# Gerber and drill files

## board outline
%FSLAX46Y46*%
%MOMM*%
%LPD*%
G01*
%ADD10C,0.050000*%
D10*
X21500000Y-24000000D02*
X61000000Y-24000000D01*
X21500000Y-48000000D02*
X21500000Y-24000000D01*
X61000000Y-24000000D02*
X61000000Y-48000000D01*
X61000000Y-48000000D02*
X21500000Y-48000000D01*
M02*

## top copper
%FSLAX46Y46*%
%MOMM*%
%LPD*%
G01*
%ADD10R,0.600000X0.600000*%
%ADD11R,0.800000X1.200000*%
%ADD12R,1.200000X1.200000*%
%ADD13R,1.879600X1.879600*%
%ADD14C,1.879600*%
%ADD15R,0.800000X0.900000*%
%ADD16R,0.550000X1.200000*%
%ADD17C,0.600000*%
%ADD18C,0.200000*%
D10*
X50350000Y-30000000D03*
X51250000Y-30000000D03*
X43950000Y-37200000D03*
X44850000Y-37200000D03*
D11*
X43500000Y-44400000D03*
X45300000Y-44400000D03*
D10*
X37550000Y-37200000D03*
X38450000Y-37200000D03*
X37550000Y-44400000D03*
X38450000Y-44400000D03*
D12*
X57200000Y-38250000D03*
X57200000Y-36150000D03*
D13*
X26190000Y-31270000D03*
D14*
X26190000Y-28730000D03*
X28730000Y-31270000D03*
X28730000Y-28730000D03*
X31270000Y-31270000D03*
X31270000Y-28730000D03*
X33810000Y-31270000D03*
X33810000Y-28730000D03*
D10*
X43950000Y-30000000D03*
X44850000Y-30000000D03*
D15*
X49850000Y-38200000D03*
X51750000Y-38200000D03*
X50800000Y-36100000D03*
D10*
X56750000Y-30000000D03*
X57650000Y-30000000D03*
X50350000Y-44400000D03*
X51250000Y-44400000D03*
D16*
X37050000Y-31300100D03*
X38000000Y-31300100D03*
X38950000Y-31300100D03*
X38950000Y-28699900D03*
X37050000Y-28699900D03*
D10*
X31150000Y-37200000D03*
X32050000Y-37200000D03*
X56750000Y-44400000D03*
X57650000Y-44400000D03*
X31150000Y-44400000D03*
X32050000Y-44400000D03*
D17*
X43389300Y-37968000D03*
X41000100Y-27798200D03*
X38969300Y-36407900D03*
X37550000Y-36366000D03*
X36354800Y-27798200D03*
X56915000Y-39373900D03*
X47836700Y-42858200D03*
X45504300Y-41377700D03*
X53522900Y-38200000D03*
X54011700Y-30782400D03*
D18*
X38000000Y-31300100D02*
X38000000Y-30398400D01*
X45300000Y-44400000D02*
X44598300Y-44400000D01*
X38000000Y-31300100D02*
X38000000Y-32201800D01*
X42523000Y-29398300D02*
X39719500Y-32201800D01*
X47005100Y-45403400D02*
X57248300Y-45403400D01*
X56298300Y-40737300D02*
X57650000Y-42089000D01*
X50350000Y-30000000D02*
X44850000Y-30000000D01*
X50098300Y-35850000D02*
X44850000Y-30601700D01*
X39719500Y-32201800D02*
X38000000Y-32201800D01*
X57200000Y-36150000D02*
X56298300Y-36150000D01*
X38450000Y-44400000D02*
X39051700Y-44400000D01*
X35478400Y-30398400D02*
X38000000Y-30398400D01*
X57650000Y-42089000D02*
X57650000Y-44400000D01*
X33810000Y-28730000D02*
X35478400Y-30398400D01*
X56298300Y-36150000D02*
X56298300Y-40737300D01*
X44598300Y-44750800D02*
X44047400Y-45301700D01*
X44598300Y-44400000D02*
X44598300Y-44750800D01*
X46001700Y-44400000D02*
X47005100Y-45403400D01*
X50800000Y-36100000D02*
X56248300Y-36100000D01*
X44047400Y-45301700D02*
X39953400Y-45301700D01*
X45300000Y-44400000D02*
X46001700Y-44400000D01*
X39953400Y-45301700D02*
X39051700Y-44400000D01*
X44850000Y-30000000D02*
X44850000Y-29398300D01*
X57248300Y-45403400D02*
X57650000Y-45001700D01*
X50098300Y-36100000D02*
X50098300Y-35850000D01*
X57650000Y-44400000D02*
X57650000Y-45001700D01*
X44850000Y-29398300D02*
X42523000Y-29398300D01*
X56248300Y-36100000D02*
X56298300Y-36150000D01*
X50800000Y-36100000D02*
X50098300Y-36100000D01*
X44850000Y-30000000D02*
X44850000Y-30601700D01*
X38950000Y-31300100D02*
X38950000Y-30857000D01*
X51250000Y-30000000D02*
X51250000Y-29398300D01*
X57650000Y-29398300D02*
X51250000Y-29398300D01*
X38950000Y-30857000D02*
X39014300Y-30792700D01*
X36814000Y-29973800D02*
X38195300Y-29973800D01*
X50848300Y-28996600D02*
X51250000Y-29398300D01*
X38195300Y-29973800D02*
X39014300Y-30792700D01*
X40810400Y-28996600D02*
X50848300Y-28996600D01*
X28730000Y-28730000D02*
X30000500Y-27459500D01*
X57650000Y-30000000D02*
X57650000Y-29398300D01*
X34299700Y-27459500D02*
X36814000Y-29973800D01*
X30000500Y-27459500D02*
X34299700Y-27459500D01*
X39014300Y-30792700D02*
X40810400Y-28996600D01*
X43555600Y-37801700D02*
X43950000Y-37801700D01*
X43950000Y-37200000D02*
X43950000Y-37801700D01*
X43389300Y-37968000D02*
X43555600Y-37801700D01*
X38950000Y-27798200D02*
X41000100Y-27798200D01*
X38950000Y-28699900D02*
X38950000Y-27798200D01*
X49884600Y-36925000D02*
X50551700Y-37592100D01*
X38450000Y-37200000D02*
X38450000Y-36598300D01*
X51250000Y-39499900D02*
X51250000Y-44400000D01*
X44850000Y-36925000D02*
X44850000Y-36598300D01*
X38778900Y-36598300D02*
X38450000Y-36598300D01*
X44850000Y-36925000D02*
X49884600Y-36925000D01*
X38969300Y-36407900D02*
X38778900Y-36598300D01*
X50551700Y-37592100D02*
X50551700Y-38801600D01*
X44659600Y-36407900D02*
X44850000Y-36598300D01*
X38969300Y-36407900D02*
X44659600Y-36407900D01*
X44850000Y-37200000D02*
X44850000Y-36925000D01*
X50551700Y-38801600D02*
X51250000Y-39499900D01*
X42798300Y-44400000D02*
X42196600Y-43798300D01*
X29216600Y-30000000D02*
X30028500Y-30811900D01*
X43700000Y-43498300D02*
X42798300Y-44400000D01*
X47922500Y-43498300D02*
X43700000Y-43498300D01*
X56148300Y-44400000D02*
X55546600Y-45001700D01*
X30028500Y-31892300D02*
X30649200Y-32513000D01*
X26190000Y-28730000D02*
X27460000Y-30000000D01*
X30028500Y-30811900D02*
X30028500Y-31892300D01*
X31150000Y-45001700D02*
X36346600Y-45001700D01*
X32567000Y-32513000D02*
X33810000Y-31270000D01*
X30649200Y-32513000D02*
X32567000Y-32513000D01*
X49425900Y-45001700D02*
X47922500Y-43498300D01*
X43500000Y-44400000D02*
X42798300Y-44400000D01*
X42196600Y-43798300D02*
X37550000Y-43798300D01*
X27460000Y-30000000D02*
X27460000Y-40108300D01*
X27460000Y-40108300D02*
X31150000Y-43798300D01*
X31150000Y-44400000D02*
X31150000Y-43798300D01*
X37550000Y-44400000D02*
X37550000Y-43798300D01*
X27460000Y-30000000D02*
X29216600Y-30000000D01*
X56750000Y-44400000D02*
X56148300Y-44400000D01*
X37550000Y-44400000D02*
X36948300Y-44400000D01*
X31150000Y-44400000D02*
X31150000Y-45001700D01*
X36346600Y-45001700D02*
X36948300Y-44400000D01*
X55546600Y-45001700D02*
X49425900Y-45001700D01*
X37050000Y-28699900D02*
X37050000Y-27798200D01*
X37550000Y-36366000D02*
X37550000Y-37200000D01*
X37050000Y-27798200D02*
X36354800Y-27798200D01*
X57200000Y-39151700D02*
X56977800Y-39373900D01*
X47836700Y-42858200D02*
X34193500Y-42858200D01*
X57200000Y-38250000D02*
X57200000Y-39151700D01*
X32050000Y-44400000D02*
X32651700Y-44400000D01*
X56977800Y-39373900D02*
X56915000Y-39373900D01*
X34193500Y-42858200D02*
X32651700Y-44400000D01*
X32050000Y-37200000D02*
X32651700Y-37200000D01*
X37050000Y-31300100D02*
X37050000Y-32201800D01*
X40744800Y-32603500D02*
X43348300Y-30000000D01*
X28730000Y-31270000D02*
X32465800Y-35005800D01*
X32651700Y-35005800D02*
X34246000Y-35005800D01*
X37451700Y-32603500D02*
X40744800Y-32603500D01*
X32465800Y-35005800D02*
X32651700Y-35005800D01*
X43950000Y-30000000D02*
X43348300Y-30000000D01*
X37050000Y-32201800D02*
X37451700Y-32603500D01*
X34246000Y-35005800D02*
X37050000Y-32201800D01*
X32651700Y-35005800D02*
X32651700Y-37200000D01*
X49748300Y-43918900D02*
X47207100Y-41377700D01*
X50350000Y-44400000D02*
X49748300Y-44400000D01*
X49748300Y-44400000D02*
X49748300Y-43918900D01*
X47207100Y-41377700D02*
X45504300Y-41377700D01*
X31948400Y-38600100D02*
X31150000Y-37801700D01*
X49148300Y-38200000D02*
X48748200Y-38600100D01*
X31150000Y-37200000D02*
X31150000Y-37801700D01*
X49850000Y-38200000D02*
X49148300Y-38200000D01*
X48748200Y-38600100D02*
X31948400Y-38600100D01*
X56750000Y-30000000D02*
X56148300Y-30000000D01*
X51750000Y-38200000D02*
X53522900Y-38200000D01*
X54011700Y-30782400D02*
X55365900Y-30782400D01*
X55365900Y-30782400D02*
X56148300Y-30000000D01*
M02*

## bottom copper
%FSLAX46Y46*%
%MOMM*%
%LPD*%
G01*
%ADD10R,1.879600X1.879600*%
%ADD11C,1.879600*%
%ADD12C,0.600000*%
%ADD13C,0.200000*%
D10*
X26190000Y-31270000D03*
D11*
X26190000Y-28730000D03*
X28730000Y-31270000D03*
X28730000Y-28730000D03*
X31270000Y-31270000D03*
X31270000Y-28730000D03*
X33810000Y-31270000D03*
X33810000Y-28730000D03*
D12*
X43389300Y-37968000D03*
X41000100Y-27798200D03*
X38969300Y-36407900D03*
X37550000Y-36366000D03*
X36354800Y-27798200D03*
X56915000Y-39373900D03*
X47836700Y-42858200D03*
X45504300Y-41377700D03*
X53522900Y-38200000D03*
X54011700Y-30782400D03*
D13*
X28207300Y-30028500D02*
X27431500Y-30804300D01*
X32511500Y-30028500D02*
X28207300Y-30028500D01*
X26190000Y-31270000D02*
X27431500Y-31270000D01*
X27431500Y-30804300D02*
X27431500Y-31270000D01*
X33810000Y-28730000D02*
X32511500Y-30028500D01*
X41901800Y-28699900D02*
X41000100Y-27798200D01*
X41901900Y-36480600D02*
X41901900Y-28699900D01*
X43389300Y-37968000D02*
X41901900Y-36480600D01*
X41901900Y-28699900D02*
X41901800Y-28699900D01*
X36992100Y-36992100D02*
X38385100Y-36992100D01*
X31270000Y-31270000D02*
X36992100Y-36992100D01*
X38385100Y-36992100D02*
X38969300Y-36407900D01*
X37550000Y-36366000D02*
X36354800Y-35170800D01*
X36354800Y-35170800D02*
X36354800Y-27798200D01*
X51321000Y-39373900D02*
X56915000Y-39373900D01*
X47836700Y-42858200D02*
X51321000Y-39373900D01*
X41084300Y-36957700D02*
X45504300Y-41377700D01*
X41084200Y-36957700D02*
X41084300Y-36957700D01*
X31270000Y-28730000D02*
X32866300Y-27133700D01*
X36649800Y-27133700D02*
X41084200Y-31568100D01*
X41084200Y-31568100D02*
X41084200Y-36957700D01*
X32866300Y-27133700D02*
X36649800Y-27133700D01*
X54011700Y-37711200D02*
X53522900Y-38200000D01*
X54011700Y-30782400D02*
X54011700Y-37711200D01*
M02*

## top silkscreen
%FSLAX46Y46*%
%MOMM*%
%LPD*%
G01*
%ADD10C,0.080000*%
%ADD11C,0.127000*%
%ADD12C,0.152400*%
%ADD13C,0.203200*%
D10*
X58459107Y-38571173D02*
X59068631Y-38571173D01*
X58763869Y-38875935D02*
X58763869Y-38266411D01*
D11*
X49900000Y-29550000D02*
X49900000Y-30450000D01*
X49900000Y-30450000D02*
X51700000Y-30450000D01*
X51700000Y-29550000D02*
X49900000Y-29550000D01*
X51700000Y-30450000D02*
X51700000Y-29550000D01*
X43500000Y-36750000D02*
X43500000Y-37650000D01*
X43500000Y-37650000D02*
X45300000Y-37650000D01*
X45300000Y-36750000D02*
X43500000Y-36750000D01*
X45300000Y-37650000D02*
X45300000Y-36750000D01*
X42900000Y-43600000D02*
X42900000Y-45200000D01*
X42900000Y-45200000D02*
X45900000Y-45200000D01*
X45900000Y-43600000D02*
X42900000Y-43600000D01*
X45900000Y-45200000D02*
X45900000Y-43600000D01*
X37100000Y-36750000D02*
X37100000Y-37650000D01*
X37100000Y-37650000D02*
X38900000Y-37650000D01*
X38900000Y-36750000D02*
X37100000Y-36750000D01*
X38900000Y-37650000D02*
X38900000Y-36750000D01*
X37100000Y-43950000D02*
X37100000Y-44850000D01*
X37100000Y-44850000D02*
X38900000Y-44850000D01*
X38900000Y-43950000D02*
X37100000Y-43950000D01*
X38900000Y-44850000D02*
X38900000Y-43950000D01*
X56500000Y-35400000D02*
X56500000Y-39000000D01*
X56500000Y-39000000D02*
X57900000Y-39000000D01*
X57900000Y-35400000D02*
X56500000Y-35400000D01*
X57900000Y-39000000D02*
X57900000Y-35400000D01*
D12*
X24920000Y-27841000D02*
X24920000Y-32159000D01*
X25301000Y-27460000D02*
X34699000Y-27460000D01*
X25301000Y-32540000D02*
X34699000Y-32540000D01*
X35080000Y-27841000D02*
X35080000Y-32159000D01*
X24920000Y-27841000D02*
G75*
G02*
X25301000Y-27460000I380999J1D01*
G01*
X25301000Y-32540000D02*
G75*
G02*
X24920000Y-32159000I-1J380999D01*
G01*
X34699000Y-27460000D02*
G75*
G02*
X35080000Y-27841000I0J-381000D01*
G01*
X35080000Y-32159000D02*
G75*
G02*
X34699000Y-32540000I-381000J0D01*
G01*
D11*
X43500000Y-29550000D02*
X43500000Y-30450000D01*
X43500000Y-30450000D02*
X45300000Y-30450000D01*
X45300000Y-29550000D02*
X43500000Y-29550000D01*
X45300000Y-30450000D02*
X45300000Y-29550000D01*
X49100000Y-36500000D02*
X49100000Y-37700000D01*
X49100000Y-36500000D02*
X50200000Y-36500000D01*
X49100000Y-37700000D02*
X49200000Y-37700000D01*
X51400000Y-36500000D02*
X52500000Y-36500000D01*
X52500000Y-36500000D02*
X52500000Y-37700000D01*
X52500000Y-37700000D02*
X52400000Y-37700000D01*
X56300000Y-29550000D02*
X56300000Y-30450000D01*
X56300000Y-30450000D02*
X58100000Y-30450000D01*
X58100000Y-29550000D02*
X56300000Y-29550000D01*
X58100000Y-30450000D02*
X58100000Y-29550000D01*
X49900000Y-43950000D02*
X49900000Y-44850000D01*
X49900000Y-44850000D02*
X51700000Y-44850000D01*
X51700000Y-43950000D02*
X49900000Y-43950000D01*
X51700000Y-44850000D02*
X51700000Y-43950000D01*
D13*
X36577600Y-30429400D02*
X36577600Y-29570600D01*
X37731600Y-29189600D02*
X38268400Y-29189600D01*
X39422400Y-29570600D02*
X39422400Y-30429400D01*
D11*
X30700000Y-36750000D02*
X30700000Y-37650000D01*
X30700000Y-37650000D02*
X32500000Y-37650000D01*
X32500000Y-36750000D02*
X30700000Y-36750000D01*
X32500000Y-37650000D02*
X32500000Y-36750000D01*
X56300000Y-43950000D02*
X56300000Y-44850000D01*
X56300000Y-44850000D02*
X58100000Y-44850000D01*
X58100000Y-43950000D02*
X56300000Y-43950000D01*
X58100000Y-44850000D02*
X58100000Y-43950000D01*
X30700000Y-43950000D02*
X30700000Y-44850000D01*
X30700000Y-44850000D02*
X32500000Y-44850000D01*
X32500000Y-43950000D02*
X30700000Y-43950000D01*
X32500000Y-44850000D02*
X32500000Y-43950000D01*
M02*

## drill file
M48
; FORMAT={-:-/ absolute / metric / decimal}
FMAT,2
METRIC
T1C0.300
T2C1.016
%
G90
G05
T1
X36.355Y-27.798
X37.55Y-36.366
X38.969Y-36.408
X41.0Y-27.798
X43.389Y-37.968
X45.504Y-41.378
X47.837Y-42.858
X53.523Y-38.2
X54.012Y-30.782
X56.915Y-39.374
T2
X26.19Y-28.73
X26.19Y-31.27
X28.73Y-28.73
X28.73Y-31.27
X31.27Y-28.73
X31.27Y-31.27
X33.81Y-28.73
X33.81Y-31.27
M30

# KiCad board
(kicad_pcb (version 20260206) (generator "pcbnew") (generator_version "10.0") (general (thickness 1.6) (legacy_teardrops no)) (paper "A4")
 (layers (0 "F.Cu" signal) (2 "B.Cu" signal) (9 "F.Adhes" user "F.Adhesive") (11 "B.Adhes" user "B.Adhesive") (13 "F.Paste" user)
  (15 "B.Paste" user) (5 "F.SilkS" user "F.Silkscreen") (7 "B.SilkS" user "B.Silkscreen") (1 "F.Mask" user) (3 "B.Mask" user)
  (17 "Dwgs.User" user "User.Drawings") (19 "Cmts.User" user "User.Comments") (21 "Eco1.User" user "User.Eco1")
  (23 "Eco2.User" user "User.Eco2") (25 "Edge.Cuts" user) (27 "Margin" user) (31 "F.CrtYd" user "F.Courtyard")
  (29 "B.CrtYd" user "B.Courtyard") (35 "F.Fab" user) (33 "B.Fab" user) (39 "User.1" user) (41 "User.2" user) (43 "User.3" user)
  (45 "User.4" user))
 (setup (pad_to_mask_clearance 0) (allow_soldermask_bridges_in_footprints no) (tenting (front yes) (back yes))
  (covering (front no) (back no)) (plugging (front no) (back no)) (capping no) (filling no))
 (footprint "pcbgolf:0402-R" (layer "F.Cu") (at 50.8 30)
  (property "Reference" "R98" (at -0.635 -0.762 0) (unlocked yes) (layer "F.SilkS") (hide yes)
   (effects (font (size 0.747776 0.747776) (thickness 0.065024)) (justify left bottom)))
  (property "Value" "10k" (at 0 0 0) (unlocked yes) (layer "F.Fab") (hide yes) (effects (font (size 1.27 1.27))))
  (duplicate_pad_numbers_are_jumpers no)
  (fp_line (start -0.9 -0.45) (end -0.9 0.45) (stroke (width 0.127) (type solid)) (layer "F.SilkS"))
  (fp_line (start -0.9 0.45) (end 0.9 0.45) (stroke (width 0.127) (type solid)) (layer "F.SilkS"))
  (fp_line (start 0.9 -0.45) (end -0.9 -0.45) (stroke (width 0.127) (type solid)) (layer "F.SilkS"))
  (fp_line (start 0.9 0.45) (end 0.9 -0.45) (stroke (width 0.127) (type solid)) (layer "F.SilkS"))
  (pad "1" smd rect (at -0.45 0) (size 0.6 0.6) (layers "F.Cu" "F.Mask" "F.Paste") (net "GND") (solder_mask_margin 0.0508)
   (solder_paste_margin 0) (thermal_bridge_angle 0))
  (pad "2" smd rect (at 0.45 0) (size 0.6 0.6) (layers "F.Cu" "F.Mask" "F.Paste") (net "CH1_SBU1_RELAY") (solder_mask_margin 0.0508)
   (solder_paste_margin 0) (thermal_bridge_angle 0)))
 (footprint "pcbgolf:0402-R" (layer "F.Cu") (at 44.4 37.2)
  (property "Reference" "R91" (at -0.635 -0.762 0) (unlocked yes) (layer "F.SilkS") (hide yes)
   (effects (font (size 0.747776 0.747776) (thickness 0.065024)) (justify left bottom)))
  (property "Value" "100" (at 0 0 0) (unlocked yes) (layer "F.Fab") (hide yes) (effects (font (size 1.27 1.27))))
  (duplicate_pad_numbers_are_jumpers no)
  (fp_line (start -0.9 -0.45) (end -0.9 0.45) (stroke (width 0.127) (type solid)) (layer "F.SilkS"))
  (fp_line (start -0.9 0.45) (end 0.9 0.45) (stroke (width 0.127) (type solid)) (layer "F.SilkS"))
  (fp_line (start 0.9 -0.45) (end -0.9 -0.45) (stroke (width 0.127) (type solid)) (layer "F.SilkS"))
  (fp_line (start 0.9 0.45) (end 0.9 -0.45) (stroke (width 0.127) (type solid)) (layer "F.SilkS"))
  (pad "1" smd rect (at -0.45 0) (size 0.6 0.6) (layers "F.Cu" "F.Mask" "F.Paste") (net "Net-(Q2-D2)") (solder_mask_margin 0.0508)
   (solder_paste_margin 0) (thermal_bridge_angle 0))
  (pad "2" smd rect (at 0.45 0) (size 0.6 0.6) (layers "F.Cu" "F.Mask" "F.Paste") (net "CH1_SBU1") (solder_mask_margin 0.0508)
   (solder_paste_margin 0) (thermal_bridge_angle 0)))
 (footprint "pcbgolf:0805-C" (layer "F.Cu") (at 44.4 44.4)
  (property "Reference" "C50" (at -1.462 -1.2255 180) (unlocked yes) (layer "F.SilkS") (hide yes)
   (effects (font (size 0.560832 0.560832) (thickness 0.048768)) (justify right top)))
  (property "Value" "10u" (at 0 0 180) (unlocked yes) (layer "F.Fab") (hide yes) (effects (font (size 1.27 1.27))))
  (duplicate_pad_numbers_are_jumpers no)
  (fp_line (start -1.5 -0.8) (end -1.5 0.8) (stroke (width 0.127) (type solid)) (layer "F.SilkS"))
  (fp_line (start -1.5 0.8) (end 1.5 0.8) (stroke (width 0.127) (type solid)) (layer "F.SilkS"))
  (fp_line (start 1.5 -0.8) (end -1.5 -0.8) (stroke (width 0.127) (type solid)) (layer "F.SilkS"))
  (fp_line (start 1.5 0.8) (end 1.5 -0.8) (stroke (width 0.127) (type solid)) (layer "F.SilkS"))
  (pad "1" smd rect (at -0.9 0) (size 0.8 1.2) (layers "F.Cu" "F.Mask" "F.Paste") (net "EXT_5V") (solder_mask_margin 0.0508)
   (solder_paste_margin 0) (thermal_bridge_angle 0))
  (pad "2" smd rect (at 0.9 0) (size 0.8 1.2) (layers "F.Cu" "F.Mask" "F.Paste") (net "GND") (solder_mask_margin 0.0508)
   (solder_paste_margin 0) (thermal_bridge_angle 0)))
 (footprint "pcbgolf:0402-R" (layer "F.Cu") (at 38 37.2)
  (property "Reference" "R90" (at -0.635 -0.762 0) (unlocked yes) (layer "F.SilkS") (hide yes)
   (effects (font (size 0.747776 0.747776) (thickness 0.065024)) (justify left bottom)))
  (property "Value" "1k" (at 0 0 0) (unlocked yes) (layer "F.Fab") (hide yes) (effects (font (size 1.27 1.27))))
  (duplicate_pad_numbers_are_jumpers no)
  (fp_line (start -0.9 -0.45) (end -0.9 0.45) (stroke (width 0.127) (type solid)) (layer "F.SilkS"))
  (fp_line (start -0.9 0.45) (end 0.9 0.45) (stroke (width 0.127) (type solid)) (layer "F.SilkS"))
  (fp_line (start 0.9 -0.45) (end -0.9 -0.45) (stroke (width 0.127) (type solid)) (layer "F.SilkS"))
  (fp_line (start 0.9 0.45) (end 0.9 -0.45) (stroke (width 0.127) (type solid)) (layer "F.SilkS"))
  (pad "1" smd rect (at -0.45 0) (size 0.6 0.6) (layers "F.Cu" "F.Mask" "F.Paste") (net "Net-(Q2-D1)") (solder_mask_margin 0.0508)
   (solder_paste_margin 0) (thermal_bridge_angle 0))
  (pad "2" smd rect (at 0.45 0) (size 0.6 0.6) (layers "F.Cu" "F.Mask" "F.Paste") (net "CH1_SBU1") (solder_mask_margin 0.0508)
   (solder_paste_margin 0) (thermal_bridge_angle 0)))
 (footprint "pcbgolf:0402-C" (layer "F.Cu") (at 38 44.4)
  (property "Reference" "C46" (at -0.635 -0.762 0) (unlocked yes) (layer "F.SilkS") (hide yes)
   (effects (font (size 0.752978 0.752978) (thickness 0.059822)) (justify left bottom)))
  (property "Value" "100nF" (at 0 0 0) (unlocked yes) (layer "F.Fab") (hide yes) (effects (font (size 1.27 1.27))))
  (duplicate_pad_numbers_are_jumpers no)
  (fp_line (start -0.9 -0.45) (end -0.9 0.45) (stroke (width 0.127) (type solid)) (layer "F.SilkS"))
  (fp_line (start -0.9 0.45) (end 0.9 0.45) (stroke (width 0.127) (type solid)) (layer "F.SilkS"))
  (fp_line (start 0.9 -0.45) (end -0.9 -0.45) (stroke (width 0.127) (type solid)) (layer "F.SilkS"))
  (fp_line (start 0.9 0.45) (end 0.9 -0.45) (stroke (width 0.127) (type solid)) (layer "F.SilkS"))
  (pad "1" smd rect (at -0.45 0) (size 0.6 0.6) (layers "F.Cu" "F.Mask" "F.Paste") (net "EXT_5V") (solder_mask_margin 0.0508)
   (solder_paste_margin 0) (thermal_bridge_angle 0))
  (pad "2" smd rect (at 0.45 0) (size 0.6 0.6) (layers "F.Cu" "F.Mask" "F.Paste") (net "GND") (solder_mask_margin 0.0508)
   (solder_paste_margin 0) (thermal_bridge_angle 0)))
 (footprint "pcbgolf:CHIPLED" (layer "F.Cu") (at 57.2 37.2)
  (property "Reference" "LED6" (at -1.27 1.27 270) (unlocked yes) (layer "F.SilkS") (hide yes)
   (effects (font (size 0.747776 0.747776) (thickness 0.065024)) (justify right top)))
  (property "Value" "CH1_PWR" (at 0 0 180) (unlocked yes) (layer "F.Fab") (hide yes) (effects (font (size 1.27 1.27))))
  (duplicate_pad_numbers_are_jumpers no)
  (fp_line (start -0.7 -1.8) (end -0.7 1.8) (stroke (width 0.127) (type solid)) (layer "F.SilkS"))
  (fp_line (start -0.7 1.8) (end 0.7 1.8) (stroke (width 0.127) (type solid)) (layer "F.SilkS"))
  (fp_line (start 0.7 -1.8) (end -0.7 -1.8) (stroke (width 0.127) (type solid)) (layer "F.SilkS"))
  (fp_line (start 0.7 1.8) (end 0.7 -1.8) (stroke (width 0.127) (type solid)) (layer "F.SilkS"))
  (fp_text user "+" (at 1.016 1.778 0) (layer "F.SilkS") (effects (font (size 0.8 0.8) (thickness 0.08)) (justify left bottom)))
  (pad "A" smd rect (at 0 1.05) (size 1.2 1.2) (layers "F.Cu" "F.Mask" "F.Paste") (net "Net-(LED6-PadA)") (solder_mask_margin 0.0508)
   (solder_paste_margin 0) (thermal_bridge_angle 0))
  (pad "C" smd rect (at 0 -1.05) (size 1.2 1.2) (layers "F.Cu" "F.Mask" "F.Paste") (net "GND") (solder_mask_margin 0.0508)
   (solder_paste_margin 0) (thermal_bridge_angle 0)))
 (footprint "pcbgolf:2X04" (layer "F.Cu") (at 30 30)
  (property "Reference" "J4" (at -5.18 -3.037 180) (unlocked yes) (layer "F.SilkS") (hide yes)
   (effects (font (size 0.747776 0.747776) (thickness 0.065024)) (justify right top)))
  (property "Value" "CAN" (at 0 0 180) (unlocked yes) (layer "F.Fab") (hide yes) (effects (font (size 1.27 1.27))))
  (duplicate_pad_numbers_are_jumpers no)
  (fp_line (start -5.08 -2.159) (end -5.08 2.159) (stroke (width 0.1524) (type solid)) (layer "F.SilkS"))
  (fp_line (start -4.699 -2.54) (end 4.699 -2.54) (stroke (width 0.1524) (type solid)) (layer "F.SilkS"))
  (fp_line (start -4.699 2.54) (end 4.699 2.54) (stroke (width 0.1524) (type solid)) (layer "F.SilkS"))
  (fp_line (start 5.08 -2.159) (end 5.08 2.159) (stroke (width 0.1524) (type solid)) (layer "F.SilkS"))
  (fp_arc (start -5.08 -2.159) (mid -4.968408 -2.428408) (end -4.699 -2.54) (stroke (width 0.1524) (type solid)) (layer "F.SilkS"))
  (fp_arc (start -4.699 2.54) (mid -4.968408 2.428408) (end -5.08 2.159) (stroke (width 0.1524) (type solid)) (layer "F.SilkS"))
  (fp_arc (start 4.699 -2.54) (mid 4.968408 -2.428408) (end 5.08 -2.159) (stroke (width 0.1524) (type solid)) (layer "F.SilkS"))
  (fp_arc (start 5.08 2.159) (mid 4.968408 2.428408) (end 4.699 2.54) (stroke (width 0.1524) (type solid)) (layer "F.SilkS"))
  (pad "1" thru_hole rect (at -3.81 1.27 90) (size 1.8796 1.8796) (drill 1.016) (layers "*.Cu" "*.Mask") (remove_unused_layers no)
   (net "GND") (solder_mask_margin 0.0508) (thermal_bridge_angle 0))
  (pad "2" thru_hole circle (at -3.81 -1.27 90) (size 1.8796 1.8796) (drill 1.016) (layers "*.Cu" "*.Mask") (remove_unused_layers no)
   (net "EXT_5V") (solder_mask_margin 0.0508) (thermal_bridge_angle 0))
  (pad "3" thru_hole circle (at -1.27 1.27 90) (size 1.8796 1.8796) (drill 1.016) (layers "*.Cu" "*.Mask") (remove_unused_layers no)
   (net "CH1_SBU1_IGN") (solder_mask_margin 0.0508) (thermal_bridge_angle 0))
  (pad "4" thru_hole circle (at -1.27 -1.27 90) (size 1.8796 1.8796) (drill 1.016) (layers "*.Cu" "*.Mask") (remove_unused_layers no)
   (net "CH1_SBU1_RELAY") (solder_mask_margin 0.0508) (thermal_bridge_angle 0))
  (pad "5" thru_hole circle (at 1.27 1.27 90) (size 1.8796 1.8796) (drill 1.016) (layers "*.Cu" "*.Mask") (remove_unused_layers no)
   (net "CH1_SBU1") (solder_mask_margin 0.0508) (thermal_bridge_angle 0))
  (pad "6" thru_hole circle (at 1.27 -1.27 90) (size 1.8796 1.8796) (drill 1.016) (layers "*.Cu" "*.Mask") (remove_unused_layers no)
   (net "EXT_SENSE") (solder_mask_margin 0.0508) (thermal_bridge_angle 0))
  (pad "7" thru_hole circle (at 3.81 1.27 90) (size 1.8796 1.8796) (drill 1.016) (layers "*.Cu" "*.Mask") (remove_unused_layers no)
   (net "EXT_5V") (solder_mask_margin 0.0508) (thermal_bridge_angle 0))
  (pad "8" thru_hole circle (at 3.81 -1.27 90) (size 1.8796 1.8796) (drill 1.016) (layers "*.Cu" "*.Mask") (remove_unused_layers no)
   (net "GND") (solder_mask_margin 0.0508) (thermal_bridge_angle 0)))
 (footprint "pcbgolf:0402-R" (layer "F.Cu") (at 44.4 30)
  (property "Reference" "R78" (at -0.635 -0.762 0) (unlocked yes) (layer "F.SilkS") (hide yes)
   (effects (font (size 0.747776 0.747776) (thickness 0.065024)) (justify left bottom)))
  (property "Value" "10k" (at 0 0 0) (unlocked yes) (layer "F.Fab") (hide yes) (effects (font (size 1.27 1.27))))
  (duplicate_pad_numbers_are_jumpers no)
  (fp_line (start -0.9 -0.45) (end -0.9 0.45) (stroke (width 0.127) (type solid)) (layer "F.SilkS"))
  (fp_line (start -0.9 0.45) (end 0.9 0.45) (stroke (width 0.127) (type solid)) (layer "F.SilkS"))
  (fp_line (start 0.9 -0.45) (end -0.9 -0.45) (stroke (width 0.127) (type solid)) (layer "F.SilkS"))
  (fp_line (start 0.9 0.45) (end 0.9 -0.45) (stroke (width 0.127) (type solid)) (layer "F.SilkS"))
  (pad "1" smd rect (at -0.45 0) (size 0.6 0.6) (layers "F.Cu" "F.Mask" "F.Paste") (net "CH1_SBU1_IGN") (solder_mask_margin 0.0508)
   (solder_paste_margin 0) (thermal_bridge_angle 0))
  (pad "2" smd rect (at 0.45 0) (size 0.6 0.6) (layers "F.Cu" "F.Mask" "F.Paste") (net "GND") (solder_mask_margin 0.0508)
   (solder_paste_margin 0) (thermal_bridge_angle 0)))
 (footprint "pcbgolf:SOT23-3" (layer "F.Cu") (at 50.8 37.2)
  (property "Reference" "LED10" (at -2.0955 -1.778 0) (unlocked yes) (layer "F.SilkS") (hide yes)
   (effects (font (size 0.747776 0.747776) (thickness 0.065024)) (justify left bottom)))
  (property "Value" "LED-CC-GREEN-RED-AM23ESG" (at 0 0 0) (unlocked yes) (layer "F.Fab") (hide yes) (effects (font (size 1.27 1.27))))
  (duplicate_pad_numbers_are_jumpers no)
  (fp_line (start -1.7 -0.7) (end -1.7 0.5) (stroke (width 0.127) (type solid)) (layer "F.SilkS"))
  (fp_line (start -1.7 -0.7) (end -0.6 -0.7) (stroke (width 0.127) (type solid)) (layer "F.SilkS"))
  (fp_line (start -1.7 0.5) (end -1.6 0.5) (stroke (width 0.127) (type solid)) (layer "F.SilkS"))
  (fp_line (start 0.6 -0.7) (end 1.7 -0.7) (stroke (width 0.127) (type solid)) (layer "F.SilkS"))
  (fp_line (start 1.7 -0.7) (end 1.7 0.5) (stroke (width 0.127) (type solid)) (layer "F.SilkS"))
  (fp_line (start 1.7 0.5) (end 1.6 0.5) (stroke (width 0.127) (type solid)) (layer "F.SilkS"))
  (pad "1" smd rect (at -0.95 1) (size 0.8 0.9) (layers "F.Cu" "F.Mask" "F.Paste") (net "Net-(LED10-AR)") (solder_mask_margin 0.0508)
   (solder_paste_margin 0) (thermal_bridge_angle 0))
  (pad "2" smd rect (at 0.95 1) (size 0.8 0.9) (layers "F.Cu" "F.Mask" "F.Paste") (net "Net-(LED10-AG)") (solder_mask_margin 0.0508)
   (solder_paste_margin 0) (thermal_bridge_angle 0))
  (pad "3" smd rect (at 0 -1.1) (size 0.8 0.9) (layers "F.Cu" "F.Mask" "F.Paste") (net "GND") (solder_mask_margin 0.0508)
   (solder_paste_margin 0) (thermal_bridge_angle 0)))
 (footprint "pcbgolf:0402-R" (layer "F.Cu") (at 57.2 30)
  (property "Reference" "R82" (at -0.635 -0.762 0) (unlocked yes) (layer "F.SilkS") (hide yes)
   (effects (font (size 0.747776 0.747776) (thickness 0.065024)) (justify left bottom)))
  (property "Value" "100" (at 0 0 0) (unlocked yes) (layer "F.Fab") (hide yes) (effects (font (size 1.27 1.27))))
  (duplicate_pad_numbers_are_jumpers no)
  (fp_line (start -0.9 -0.45) (end -0.9 0.45) (stroke (width 0.127) (type solid)) (layer "F.SilkS"))
  (fp_line (start -0.9 0.45) (end 0.9 0.45) (stroke (width 0.127) (type solid)) (layer "F.SilkS"))
  (fp_line (start 0.9 -0.45) (end -0.9 -0.45) (stroke (width 0.127) (type solid)) (layer "F.SilkS"))
  (fp_line (start 0.9 0.45) (end 0.9 -0.45) (stroke (width 0.127) (type solid)) (layer "F.SilkS"))
  (pad "1" smd rect (at -0.45 0) (size 0.6 0.6) (layers "F.Cu" "F.Mask" "F.Paste") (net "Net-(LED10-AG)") (solder_mask_margin 0.0508)
   (solder_paste_margin 0) (thermal_bridge_angle 0))
  (pad "2" smd rect (at 0.45 0) (size 0.6 0.6) (layers "F.Cu" "F.Mask" "F.Paste") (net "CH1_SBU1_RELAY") (solder_mask_margin 0.0508)
   (solder_paste_margin 0) (thermal_bridge_angle 0)))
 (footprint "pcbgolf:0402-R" (layer "F.Cu") (at 50.8 44.4)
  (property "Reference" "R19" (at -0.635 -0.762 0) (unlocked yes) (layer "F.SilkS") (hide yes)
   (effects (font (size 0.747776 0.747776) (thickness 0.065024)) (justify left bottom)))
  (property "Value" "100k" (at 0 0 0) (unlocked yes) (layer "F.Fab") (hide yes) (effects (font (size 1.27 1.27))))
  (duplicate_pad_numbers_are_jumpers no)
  (fp_line (start -0.9 -0.45) (end -0.9 0.45) (stroke (width 0.127) (type solid)) (layer "F.SilkS"))
  (fp_line (start -0.9 0.45) (end 0.9 0.45) (stroke (width 0.127) (type solid)) (layer "F.SilkS"))
  (fp_line (start 0.9 -0.45) (end -0.9 -0.45) (stroke (width 0.127) (type solid)) (layer "F.SilkS"))
  (fp_line (start 0.9 0.45) (end 0.9 -0.45) (stroke (width 0.127) (type solid)) (layer "F.SilkS"))
  (pad "1" smd rect (at -0.45 0) (size 0.6 0.6) (layers "F.Cu" "F.Mask" "F.Paste") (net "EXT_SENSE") (solder_mask_margin 0.0508)
   (solder_paste_margin 0) (thermal_bridge_angle 0))
  (pad "2" smd rect (at 0.45 0) (size 0.6 0.6) (layers "F.Cu" "F.Mask" "F.Paste") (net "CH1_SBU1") (solder_mask_margin 0.0508)
   (solder_paste_margin 0) (thermal_bridge_angle 0)))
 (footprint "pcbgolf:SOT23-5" (layer "F.Cu") (at 38 30)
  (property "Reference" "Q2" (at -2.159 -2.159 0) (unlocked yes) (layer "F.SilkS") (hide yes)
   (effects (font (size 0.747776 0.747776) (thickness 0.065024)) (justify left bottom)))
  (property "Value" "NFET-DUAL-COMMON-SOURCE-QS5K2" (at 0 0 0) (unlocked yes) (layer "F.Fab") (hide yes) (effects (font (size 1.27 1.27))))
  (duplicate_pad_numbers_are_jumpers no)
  (fp_line (start -1.4224 0.4294) (end -1.4224 -0.4294) (stroke (width 0.2032) (type solid)) (layer "F.SilkS"))
  (fp_line (start -0.2684 -0.8104) (end 0.2684 -0.8104) (stroke (width 0.2032) (type solid)) (layer "F.SilkS"))
  (fp_line (start 1.4224 -0.4294) (end 1.4224 0.4294) (stroke (width 0.2032) (type solid)) (layer "F.SilkS"))
  (pad "1" smd rect (at -0.95 1.3001) (size 0.55 1.2) (layers "F.Cu" "F.Mask" "F.Paste") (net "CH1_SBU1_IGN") (solder_mask_margin 0.0508)
   (solder_paste_margin 0) (thermal_bridge_angle 0))
  (pad "2" smd rect (at 0 1.3001) (size 0.55 1.2) (layers "F.Cu" "F.Mask" "F.Paste") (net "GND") (solder_mask_margin 0.0508)
   (solder_paste_margin 0) (thermal_bridge_angle 0))
  (pad "3" smd rect (at 0.95 1.3001) (size 0.55 1.2) (layers "F.Cu" "F.Mask" "F.Paste") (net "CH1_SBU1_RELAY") (solder_mask_margin 0.0508)
   (solder_paste_margin 0) (thermal_bridge_angle 0))
  (pad "4" smd rect (at 0.95 -1.3001) (size 0.55 1.2) (layers "F.Cu" "F.Mask" "F.Paste") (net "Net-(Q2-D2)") (solder_mask_margin 0.0508)
   (solder_paste_margin 0) (thermal_bridge_angle 0))
  (pad "5" smd rect (at -0.95 -1.3001) (size 0.55 1.2) (layers "F.Cu" "F.Mask" "F.Paste") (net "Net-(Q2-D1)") (solder_mask_margin 0.0508)
   (solder_paste_margin 0) (thermal_bridge_angle 0)))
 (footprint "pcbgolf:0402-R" (layer "F.Cu") (at 31.6 37.2)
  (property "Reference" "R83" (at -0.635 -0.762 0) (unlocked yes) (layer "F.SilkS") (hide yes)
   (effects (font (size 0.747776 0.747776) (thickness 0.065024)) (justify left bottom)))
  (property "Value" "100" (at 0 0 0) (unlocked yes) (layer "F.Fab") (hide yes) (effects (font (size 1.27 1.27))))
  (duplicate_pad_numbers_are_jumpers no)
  (fp_line (start -0.9 -0.45) (end -0.9 0.45) (stroke (width 0.127) (type solid)) (layer "F.SilkS"))
  (fp_line (start -0.9 0.45) (end 0.9 0.45) (stroke (width 0.127) (type solid)) (layer "F.SilkS"))
  (fp_line (start 0.9 -0.45) (end -0.9 -0.45) (stroke (width 0.127) (type solid)) (layer "F.SilkS"))
  (fp_line (start 0.9 0.45) (end 0.9 -0.45) (stroke (width 0.127) (type solid)) (layer "F.SilkS"))
  (pad "1" smd rect (at -0.45 0) (size 0.6 0.6) (layers "F.Cu" "F.Mask" "F.Paste") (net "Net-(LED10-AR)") (solder_mask_margin 0.0508)
   (solder_paste_margin 0) (thermal_bridge_angle 0))
  (pad "2" smd rect (at 0.45 0) (size 0.6 0.6) (layers "F.Cu" "F.Mask" "F.Paste") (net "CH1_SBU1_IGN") (solder_mask_margin 0.0508)
   (solder_paste_margin 0) (thermal_bridge_angle 0)))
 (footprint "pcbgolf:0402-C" (layer "F.Cu") (at 57.2 44.4)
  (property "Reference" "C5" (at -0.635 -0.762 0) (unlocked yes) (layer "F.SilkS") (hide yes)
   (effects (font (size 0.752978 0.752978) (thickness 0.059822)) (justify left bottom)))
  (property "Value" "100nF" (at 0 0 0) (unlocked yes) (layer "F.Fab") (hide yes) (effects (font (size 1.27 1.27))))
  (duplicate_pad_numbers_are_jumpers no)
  (fp_line (start -0.9 -0.45) (end -0.9 0.45) (stroke (width 0.127) (type solid)) (layer "F.SilkS"))
  (fp_line (start -0.9 0.45) (end 0.9 0.45) (stroke (width 0.127) (type solid)) (layer "F.SilkS"))
  (fp_line (start 0.9 -0.45) (end -0.9 -0.45) (stroke (width 0.127) (type solid)) (layer "F.SilkS"))
  (fp_line (start 0.9 0.45) (end 0.9 -0.45) (stroke (width 0.127) (type solid)) (layer "F.SilkS"))
  (pad "1" smd rect (at -0.45 0) (size 0.6 0.6) (layers "F.Cu" "F.Mask" "F.Paste") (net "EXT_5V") (solder_mask_margin 0.0508)
   (solder_paste_margin 0) (thermal_bridge_angle 0))
  (pad "2" smd rect (at 0.45 0) (size 0.6 0.6) (layers "F.Cu" "F.Mask" "F.Paste") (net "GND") (solder_mask_margin 0.0508)
   (solder_paste_margin 0) (thermal_bridge_angle 0)))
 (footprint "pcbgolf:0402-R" (layer "F.Cu") (at 31.6 44.4)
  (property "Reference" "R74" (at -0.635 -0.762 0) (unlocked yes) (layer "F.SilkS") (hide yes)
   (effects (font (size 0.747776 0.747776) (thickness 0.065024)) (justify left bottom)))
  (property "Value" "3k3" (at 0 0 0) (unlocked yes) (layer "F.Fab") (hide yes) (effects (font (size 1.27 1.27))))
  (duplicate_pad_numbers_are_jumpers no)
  (fp_line (start -0.9 -0.45) (end -0.9 0.45) (stroke (width 0.127) (type solid)) (layer "F.SilkS"))
  (fp_line (start -0.9 0.45) (end 0.9 0.45) (stroke (width 0.127) (type solid)) (layer "F.SilkS"))
  (fp_line (start 0.9 -0.45) (end -0.9 -0.45) (stroke (width 0.127) (type solid)) (layer "F.SilkS"))
  (fp_line (start 0.9 0.45) (end 0.9 -0.45) (stroke (width 0.127) (type solid)) (layer "F.SilkS"))
  (pad "1" smd rect (at -0.45 0) (size 0.6 0.6) (layers "F.Cu" "F.Mask" "F.Paste") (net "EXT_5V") (solder_mask_margin 0.0508)
   (solder_paste_margin 0) (thermal_bridge_angle 0))
  (pad "2" smd rect (at 0.45 0) (size 0.6 0.6) (layers "F.Cu" "F.Mask" "F.Paste") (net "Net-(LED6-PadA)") (solder_mask_margin 0.0508)
   (solder_paste_margin 0) (thermal_bridge_angle 0)))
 (gr_line (start 21.5 24) (end 61 24) (stroke (width 0.05) (type default)) (layer "Edge.Cuts"))
 (gr_line (start 21.5 48) (end 21.5 24) (stroke (width 0.05) (type default)) (layer "Edge.Cuts"))
 (gr_line (start 61 24) (end 61 48) (stroke (width 0.05) (type default)) (layer "Edge.Cuts"))
 (gr_line (start 61 48) (end 21.5 48) (stroke (width 0.05) (type default)) (layer "Edge.Cuts"))
 (segment (start 38 31.3001) (end 38 30.3984) (width 0.2) (layer "F.Cu") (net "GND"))
 (segment (start 45.3 44.4) (end 44.5983 44.4) (width 0.2) (layer "F.Cu") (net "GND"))
 (segment (start 38 31.3001) (end 38 32.2018) (width 0.2) (layer "F.Cu") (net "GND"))
 (segment (start 42.523 29.3983) (end 39.7195 32.2018) (width 0.2) (layer "F.Cu") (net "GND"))
 (segment (start 47.0051 45.4034) (end 57.2483 45.4034) (width 0.2) (layer "F.Cu") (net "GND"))
 (segment (start 56.2983 40.7373) (end 57.65 42.089) (width 0.2) (layer "F.Cu") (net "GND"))
 (segment (start 50.35 30) (end 44.85 30) (width 0.2) (layer "F.Cu") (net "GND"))
 (segment (start 50.0983 35.85) (end 44.85 30.6017) (width 0.2) (layer "F.Cu") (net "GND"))
 (segment (start 39.7195 32.2018) (end 38 32.2018) (width 0.2) (layer "F.Cu") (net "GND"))
 (segment (start 57.2 36.15) (end 56.2983 36.15) (width 0.2) (layer "F.Cu") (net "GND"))
 (segment (start 38.45 44.4) (end 39.0517 44.4) (width 0.2) (layer "F.Cu") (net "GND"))
 (segment (start 35.4784 30.3984) (end 38 30.3984) (width 0.2) (layer "F.Cu") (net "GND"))
 (segment (start 57.65 42.089) (end 57.65 44.4) (width 0.2) (layer "F.Cu") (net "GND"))
 (segment (start 33.81 28.73) (end 35.4784 30.3984) (width 0.2) (layer "F.Cu") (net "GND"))
 (segment (start 56.2983 36.15) (end 56.2983 40.7373) (width 0.2) (layer "F.Cu") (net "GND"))
 (segment (start 44.5983 44.7508) (end 44.0474 45.3017) (width 0.2) (layer "F.Cu") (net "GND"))
 (segment (start 44.5983 44.4) (end 44.5983 44.7508) (width 0.2) (layer "F.Cu") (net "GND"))
 (segment (start 46.0017 44.4) (end 47.0051 45.4034) (width 0.2) (layer "F.Cu") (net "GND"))
 (segment (start 50.8 36.1) (end 56.2483 36.1) (width 0.2) (layer "F.Cu") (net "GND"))
 (segment (start 44.0474 45.3017) (end 39.9534 45.3017) (width 0.2) (layer "F.Cu") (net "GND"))
 (segment (start 45.3 44.4) (end 46.0017 44.4) (width 0.2) (layer "F.Cu") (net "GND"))
 (segment (start 39.9534 45.3017) (end 39.0517 44.4) (width 0.2) (layer "F.Cu") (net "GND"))
 (segment (start 44.85 30) (end 44.85 29.3983) (width 0.2) (layer "F.Cu") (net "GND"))
 (segment (start 57.2483 45.4034) (end 57.65 45.0017) (width 0.2) (layer "F.Cu") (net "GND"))
 (segment (start 50.0983 36.1) (end 50.0983 35.85) (width 0.2) (layer "F.Cu") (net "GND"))
 (segment (start 57.65 44.4) (end 57.65 45.0017) (width 0.2) (layer "F.Cu") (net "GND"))
 (segment (start 44.85 29.3983) (end 42.523 29.3983) (width 0.2) (layer "F.Cu") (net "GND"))
 (segment (start 56.2483 36.1) (end 56.2983 36.15) (width 0.2) (layer "F.Cu") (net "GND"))
 (segment (start 50.8 36.1) (end 50.0983 36.1) (width 0.2) (layer "F.Cu") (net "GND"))
 (segment (start 44.85 30) (end 44.85 30.6017) (width 0.2) (layer "F.Cu") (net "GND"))
 (segment (start 28.2073 30.0285) (end 27.4315 30.8043) (width 0.2) (layer "B.Cu") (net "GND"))
 (segment (start 32.5115 30.0285) (end 28.2073 30.0285) (width 0.2) (layer "B.Cu") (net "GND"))
 (segment (start 26.19 31.27) (end 27.4315 31.27) (width 0.2) (layer "B.Cu") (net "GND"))
 (segment (start 27.4315 30.8043) (end 27.4315 31.27) (width 0.2) (layer "B.Cu") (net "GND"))
 (segment (start 33.81 28.73) (end 32.5115 30.0285) (width 0.2) (layer "B.Cu") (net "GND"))
 (segment (start 38.95 31.3001) (end 38.95 30.857) (width 0.2) (layer "F.Cu") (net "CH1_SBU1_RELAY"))
 (segment (start 51.25 30) (end 51.25 29.3983) (width 0.2) (layer "F.Cu") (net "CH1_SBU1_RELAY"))
 (segment (start 57.65 29.3983) (end 51.25 29.3983) (width 0.2) (layer "F.Cu") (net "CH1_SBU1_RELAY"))
 (segment (start 38.95 30.857) (end 39.0143 30.7927) (width 0.2) (layer "F.Cu") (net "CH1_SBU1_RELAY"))
 (segment (start 36.814 29.9738) (end 38.1953 29.9738) (width 0.2) (layer "F.Cu") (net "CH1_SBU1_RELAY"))
 (segment (start 50.8483 28.9966) (end 51.25 29.3983) (width 0.2) (layer "F.Cu") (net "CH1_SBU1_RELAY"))
 (segment (start 38.1953 29.9738) (end 39.0143 30.7927) (width 0.2) (layer "F.Cu") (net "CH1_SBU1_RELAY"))
 (segment (start 40.8104 28.9966) (end 50.8483 28.9966) (width 0.2) (layer "F.Cu") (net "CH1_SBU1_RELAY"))
 (segment (start 28.73 28.73) (end 30.0005 27.4595) (width 0.2) (layer "F.Cu") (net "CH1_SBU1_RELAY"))
 (segment (start 57.65 30) (end 57.65 29.3983) (width 0.2) (layer "F.Cu") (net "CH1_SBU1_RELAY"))
 (segment (start 34.2997 27.4595) (end 36.814 29.9738) (width 0.2) (layer "F.Cu") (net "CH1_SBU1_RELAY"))
 (segment (start 30.0005 27.4595) (end 34.2997 27.4595) (width 0.2) (layer "F.Cu") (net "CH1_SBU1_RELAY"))
 (segment (start 39.0143 30.7927) (end 40.8104 28.9966) (width 0.2) (layer "F.Cu") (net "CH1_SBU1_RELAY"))
 (segment (start 43.5556 37.8017) (end 43.95 37.8017) (width 0.2) (layer "F.Cu") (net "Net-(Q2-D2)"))
 (segment (start 43.95 37.2) (end 43.95 37.8017) (width 0.2) (layer "F.Cu") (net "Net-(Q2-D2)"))
 (segment (start 43.3893 37.968) (end 43.5556 37.8017) (width 0.2) (layer "F.Cu") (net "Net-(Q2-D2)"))
 (segment (start 38.95 27.7982) (end 41.0001 27.7982) (width 0.2) (layer "F.Cu") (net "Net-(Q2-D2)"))
 (segment (start 38.95 28.6999) (end 38.95 27.7982) (width 0.2) (layer "F.Cu") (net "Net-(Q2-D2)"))
 (via (at 43.3893 37.968) (size 0.6) (drill 0.3) (layers "F.Cu" "B.Cu") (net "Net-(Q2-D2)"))
 (via (at 41.0001 27.7982) (size 0.6) (drill 0.3) (layers "F.Cu" "B.Cu") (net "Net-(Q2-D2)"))
 (segment (start 41.9018 28.6999) (end 41.0001 27.7982) (width 0.2) (layer "B.Cu") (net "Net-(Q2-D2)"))
 (segment (start 41.9019 36.4806) (end 41.9019 28.6999) (width 0.2) (layer "B.Cu") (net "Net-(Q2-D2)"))
 (segment (start 43.3893 37.968) (end 41.9019 36.4806) (width 0.2) (layer "B.Cu") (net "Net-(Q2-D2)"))
 (segment (start 41.9019 28.6999) (end 41.9018 28.6999) (width 0.2) (layer "B.Cu") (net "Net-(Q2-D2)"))
 (segment (start 49.8846 36.925) (end 50.5517 37.5921) (width 0.2) (layer "F.Cu") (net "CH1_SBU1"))
 (segment (start 38.45 37.2) (end 38.45 36.5983) (width 0.2) (layer "F.Cu") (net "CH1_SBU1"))
 (segment (start 51.25 39.4999) (end 51.25 44.4) (width 0.2) (layer "F.Cu") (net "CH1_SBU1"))
 (segment (start 44.85 36.925) (end 44.85 36.5983) (width 0.2) (layer "F.Cu") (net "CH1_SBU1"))
 (segment (start 38.7789 36.5983) (end 38.45 36.5983) (width 0.2) (layer "F.Cu") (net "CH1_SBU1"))
 (segment (start 44.85 36.925) (end 49.8846 36.925) (width 0.2) (layer "F.Cu") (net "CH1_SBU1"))
 (segment (start 38.9693 36.4079) (end 38.7789 36.5983) (width 0.2) (layer "F.Cu") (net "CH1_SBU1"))
 (segment (start 50.5517 37.5921) (end 50.5517 38.8016) (width 0.2) (layer "F.Cu") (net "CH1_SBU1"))
 (segment (start 44.6596 36.4079) (end 44.85 36.5983) (width 0.2) (layer "F.Cu") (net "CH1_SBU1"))
 (segment (start 38.9693 36.4079) (end 44.6596 36.4079) (width 0.2) (layer "F.Cu") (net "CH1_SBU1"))
 (segment (start 44.85 37.2) (end 44.85 36.925) (width 0.2) (layer "F.Cu") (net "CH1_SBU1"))
 (segment (start 50.5517 38.8016) (end 51.25 39.4999) (width 0.2) (layer "F.Cu") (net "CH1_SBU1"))
 (via (at 38.9693 36.4079) (size 0.6) (drill 0.3) (layers "F.Cu" "B.Cu") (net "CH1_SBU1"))
 (segment (start 36.9921 36.9921) (end 38.3851 36.9921) (width 0.2) (layer "B.Cu") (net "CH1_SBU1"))
 (segment (start 31.27 31.27) (end 36.9921 36.9921) (width 0.2) (layer "B.Cu") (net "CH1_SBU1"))
 (segment (start 38.3851 36.9921) (end 38.9693 36.4079) (width 0.2) (layer "B.Cu") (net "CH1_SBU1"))
 (segment (start 42.7983 44.4) (end 42.1966 43.7983) (width 0.2) (layer "F.Cu") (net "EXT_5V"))
 (segment (start 29.2166 30) (end 30.0285 30.8119) (width 0.2) (layer "F.Cu") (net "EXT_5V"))
 (segment (start 43.7 43.4983) (end 42.7983 44.4) (width 0.2) (layer "F.Cu") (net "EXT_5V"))
 (segment (start 47.9225 43.4983) (end 43.7 43.4983) (width 0.2) (layer "F.Cu") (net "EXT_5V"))
 (segment (start 56.1483 44.4) (end 55.5466 45.0017) (width 0.2) (layer "F.Cu") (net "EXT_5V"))
 (segment (start 30.0285 31.8923) (end 30.6492 32.513) (width 0.2) (layer "F.Cu") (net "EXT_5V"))
 (segment (start 26.19 28.73) (end 27.46 30) (width 0.2) (layer "F.Cu") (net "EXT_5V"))
 (segment (start 30.0285 30.8119) (end 30.0285 31.8923) (width 0.2) (layer "F.Cu") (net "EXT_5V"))
 (segment (start 31.15 45.0017) (end 36.3466 45.0017) (width 0.2) (layer "F.Cu") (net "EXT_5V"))
 (segment (start 32.567 32.513) (end 33.81 31.27) (width 0.2) (layer "F.Cu") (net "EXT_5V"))
 (segment (start 30.6492 32.513) (end 32.567 32.513) (width 0.2) (layer "F.Cu") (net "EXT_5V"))
 (segment (start 49.4259 45.0017) (end 47.9225 43.4983) (width 0.2) (layer "F.Cu") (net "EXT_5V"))
 (segment (start 43.5 44.4) (end 42.7983 44.4) (width 0.2) (layer "F.Cu") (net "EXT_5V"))
 (segment (start 42.1966 43.7983) (end 37.55 43.7983) (width 0.2) (layer "F.Cu") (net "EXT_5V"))
 (segment (start 27.46 30) (end 27.46 40.1083) (width 0.2) (layer "F.Cu") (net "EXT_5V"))
 (segment (start 27.46 40.1083) (end 31.15 43.7983) (width 0.2) (layer "F.Cu") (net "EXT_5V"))
 (segment (start 31.15 44.4) (end 31.15 43.7983) (width 0.2) (layer "F.Cu") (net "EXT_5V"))
 (segment (start 37.55 44.4) (end 37.55 43.7983) (width 0.2) (layer "F.Cu") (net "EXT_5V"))
 (segment (start 27.46 30) (end 29.2166 30) (width 0.2) (layer "F.Cu") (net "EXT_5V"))
 (segment (start 56.75 44.4) (end 56.1483 44.4) (width 0.2) (layer "F.Cu") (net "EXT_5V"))
 (segment (start 37.55 44.4) (end 36.9483 44.4) (width 0.2) (layer "F.Cu") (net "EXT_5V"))
 (segment (start 31.15 44.4) (end 31.15 45.0017) (width 0.2) (layer "F.Cu") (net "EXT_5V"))
 (segment (start 36.3466 45.0017) (end 36.9483 44.4) (width 0.2) (layer "F.Cu") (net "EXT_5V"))
 (segment (start 55.5466 45.0017) (end 49.4259 45.0017) (width 0.2) (layer "F.Cu") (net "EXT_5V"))
 (segment (start 37.05 28.6999) (end 37.05 27.7982) (width 0.2) (layer "F.Cu") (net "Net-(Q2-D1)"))
 (segment (start 37.55 36.366) (end 37.55 37.2) (width 0.2) (layer "F.Cu") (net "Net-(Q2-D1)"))
 (segment (start 37.05 27.7982) (end 36.3548 27.7982) (width 0.2) (layer "F.Cu") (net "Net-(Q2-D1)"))
 (via (at 37.55 36.366) (size 0.6) (drill 0.3) (layers "F.Cu" "B.Cu") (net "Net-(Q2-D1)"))
 (via (at 36.3548 27.7982) (size 0.6) (drill 0.3) (layers "F.Cu" "B.Cu") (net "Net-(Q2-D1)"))
 (segment (start 37.55 36.366) (end 36.3548 35.1708) (width 0.2) (layer "B.Cu") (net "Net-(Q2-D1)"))
 (segment (start 36.3548 35.1708) (end 36.3548 27.7982) (width 0.2) (layer "B.Cu") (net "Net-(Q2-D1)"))
 (segment (start 57.2 39.1517) (end 56.9778 39.3739) (width 0.2) (layer "F.Cu") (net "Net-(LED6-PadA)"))
 (segment (start 47.8367 42.8582) (end 34.1935 42.8582) (width 0.2) (layer "F.Cu") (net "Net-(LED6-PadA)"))
 (segment (start 57.2 38.25) (end 57.2 39.1517) (width 0.2) (layer "F.Cu") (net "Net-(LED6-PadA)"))
 (segment (start 32.05 44.4) (end 32.6517 44.4) (width 0.2) (layer "F.Cu") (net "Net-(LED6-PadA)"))
 (segment (start 56.9778 39.3739) (end 56.915 39.3739) (width 0.2) (layer "F.Cu") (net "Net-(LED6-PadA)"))
 (segment (start 34.1935 42.8582) (end 32.6517 44.4) (width 0.2) (layer "F.Cu") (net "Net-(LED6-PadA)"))
 (via (at 56.915 39.3739) (size 0.6) (drill 0.3) (layers "F.Cu" "B.Cu") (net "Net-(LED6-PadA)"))
 (via (at 47.8367 42.8582) (size 0.6) (drill 0.3) (layers "F.Cu" "B.Cu") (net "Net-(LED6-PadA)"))
 (segment (start 51.321 39.3739) (end 56.915 39.3739) (width 0.2) (layer "B.Cu") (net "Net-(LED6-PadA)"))
 (segment (start 47.8367 42.8582) (end 51.321 39.3739) (width 0.2) (layer "B.Cu") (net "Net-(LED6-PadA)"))
 (segment (start 32.05 37.2) (end 32.6517 37.2) (width 0.2) (layer "F.Cu") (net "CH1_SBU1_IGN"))
 (segment (start 37.05 31.3001) (end 37.05 32.2018) (width 0.2) (layer "F.Cu") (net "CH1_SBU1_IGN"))
 (segment (start 40.7448 32.6035) (end 43.3483 30) (width 0.2) (layer "F.Cu") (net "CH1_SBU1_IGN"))
 (segment (start 28.73 31.27) (end 32.4658 35.0058) (width 0.2) (layer "F.Cu") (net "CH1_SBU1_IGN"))
 (segment (start 32.6517 35.0058) (end 34.246 35.0058) (width 0.2) (layer "F.Cu") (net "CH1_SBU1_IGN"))
 (segment (start 37.4517 32.6035) (end 40.7448 32.6035) (width 0.2) (layer "F.Cu") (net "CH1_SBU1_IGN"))
 (segment (start 32.4658 35.0058) (end 32.6517 35.0058) (width 0.2) (layer "F.Cu") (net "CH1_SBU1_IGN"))
 (segment (start 43.95 30) (end 43.3483 30) (width 0.2) (layer "F.Cu") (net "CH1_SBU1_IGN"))
 (segment (start 37.05 32.2018) (end 37.4517 32.6035) (width 0.2) (layer "F.Cu") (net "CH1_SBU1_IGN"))
 (segment (start 34.246 35.0058) (end 37.05 32.2018) (width 0.2) (layer "F.Cu") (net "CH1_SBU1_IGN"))
 (segment (start 32.6517 35.0058) (end 32.6517 37.2) (width 0.2) (layer "F.Cu") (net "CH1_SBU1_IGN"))
 (segment (start 49.7483 43.9189) (end 47.2071 41.3777) (width 0.2) (layer "F.Cu") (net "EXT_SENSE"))
 (segment (start 50.35 44.4) (end 49.7483 44.4) (width 0.2) (layer "F.Cu") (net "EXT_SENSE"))
 (segment (start 49.7483 44.4) (end 49.7483 43.9189) (width 0.2) (layer "F.Cu") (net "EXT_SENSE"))
 (segment (start 47.2071 41.3777) (end 45.5043 41.3777) (width 0.2) (layer "F.Cu") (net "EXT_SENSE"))
 (via (at 45.5043 41.3777) (size 0.6) (drill 0.3) (layers "F.Cu" "B.Cu") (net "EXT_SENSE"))
 (segment (start 41.0843 36.9577) (end 45.5043 41.3777) (width 0.2) (layer "B.Cu") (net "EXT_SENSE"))
 (segment (start 41.0842 36.9577) (end 41.0843 36.9577) (width 0.2) (layer "B.Cu") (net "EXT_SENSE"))
 (segment (start 31.27 28.73) (end 32.8663 27.1337) (width 0.2) (layer "B.Cu") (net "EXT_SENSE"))
 (segment (start 36.6498 27.1337) (end 41.0842 31.5681) (width 0.2) (layer "B.Cu") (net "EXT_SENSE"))
 (segment (start 41.0842 31.5681) (end 41.0842 36.9577) (width 0.2) (layer "B.Cu") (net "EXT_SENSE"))
 (segment (start 32.8663 27.1337) (end 36.6498 27.1337) (width 0.2) (layer "B.Cu") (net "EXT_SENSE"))
 (segment (start 31.9484 38.6001) (end 31.15 37.8017) (width 0.2) (layer "F.Cu") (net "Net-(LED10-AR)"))
 (segment (start 49.1483 38.2) (end 48.7482 38.6001) (width 0.2) (layer "F.Cu") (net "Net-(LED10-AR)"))
 (segment (start 31.15 37.2) (end 31.15 37.8017) (width 0.2) (layer "F.Cu") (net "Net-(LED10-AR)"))
 (segment (start 49.85 38.2) (end 49.1483 38.2) (width 0.2) (layer "F.Cu") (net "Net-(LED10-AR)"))
 (segment (start 48.7482 38.6001) (end 31.9484 38.6001) (width 0.2) (layer "F.Cu") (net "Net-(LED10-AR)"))
 (segment (start 56.75 30) (end 56.1483 30) (width 0.2) (layer "F.Cu") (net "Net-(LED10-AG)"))
 (segment (start 51.75 38.2) (end 53.5229 38.2) (width 0.2) (layer "F.Cu") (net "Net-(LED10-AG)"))
 (segment (start 54.0117 30.7824) (end 55.3659 30.7824) (width 0.2) (layer "F.Cu") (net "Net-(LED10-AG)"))
 (segment (start 55.3659 30.7824) (end 56.1483 30) (width 0.2) (layer "F.Cu") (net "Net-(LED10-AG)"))
 (via (at 53.5229 38.2) (size 0.6) (drill 0.3) (layers "F.Cu" "B.Cu") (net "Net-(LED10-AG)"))
 (via (at 54.0117 30.7824) (size 0.6) (drill 0.3) (layers "F.Cu" "B.Cu") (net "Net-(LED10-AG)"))
 (segment (start 54.0117 37.7112) (end 53.5229 38.2) (width 0.2) (layer "B.Cu") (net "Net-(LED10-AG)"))
 (segment (start 54.0117 30.7824) (end 54.0117 37.7112) (width 0.2) (layer "B.Cu") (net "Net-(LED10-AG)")))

